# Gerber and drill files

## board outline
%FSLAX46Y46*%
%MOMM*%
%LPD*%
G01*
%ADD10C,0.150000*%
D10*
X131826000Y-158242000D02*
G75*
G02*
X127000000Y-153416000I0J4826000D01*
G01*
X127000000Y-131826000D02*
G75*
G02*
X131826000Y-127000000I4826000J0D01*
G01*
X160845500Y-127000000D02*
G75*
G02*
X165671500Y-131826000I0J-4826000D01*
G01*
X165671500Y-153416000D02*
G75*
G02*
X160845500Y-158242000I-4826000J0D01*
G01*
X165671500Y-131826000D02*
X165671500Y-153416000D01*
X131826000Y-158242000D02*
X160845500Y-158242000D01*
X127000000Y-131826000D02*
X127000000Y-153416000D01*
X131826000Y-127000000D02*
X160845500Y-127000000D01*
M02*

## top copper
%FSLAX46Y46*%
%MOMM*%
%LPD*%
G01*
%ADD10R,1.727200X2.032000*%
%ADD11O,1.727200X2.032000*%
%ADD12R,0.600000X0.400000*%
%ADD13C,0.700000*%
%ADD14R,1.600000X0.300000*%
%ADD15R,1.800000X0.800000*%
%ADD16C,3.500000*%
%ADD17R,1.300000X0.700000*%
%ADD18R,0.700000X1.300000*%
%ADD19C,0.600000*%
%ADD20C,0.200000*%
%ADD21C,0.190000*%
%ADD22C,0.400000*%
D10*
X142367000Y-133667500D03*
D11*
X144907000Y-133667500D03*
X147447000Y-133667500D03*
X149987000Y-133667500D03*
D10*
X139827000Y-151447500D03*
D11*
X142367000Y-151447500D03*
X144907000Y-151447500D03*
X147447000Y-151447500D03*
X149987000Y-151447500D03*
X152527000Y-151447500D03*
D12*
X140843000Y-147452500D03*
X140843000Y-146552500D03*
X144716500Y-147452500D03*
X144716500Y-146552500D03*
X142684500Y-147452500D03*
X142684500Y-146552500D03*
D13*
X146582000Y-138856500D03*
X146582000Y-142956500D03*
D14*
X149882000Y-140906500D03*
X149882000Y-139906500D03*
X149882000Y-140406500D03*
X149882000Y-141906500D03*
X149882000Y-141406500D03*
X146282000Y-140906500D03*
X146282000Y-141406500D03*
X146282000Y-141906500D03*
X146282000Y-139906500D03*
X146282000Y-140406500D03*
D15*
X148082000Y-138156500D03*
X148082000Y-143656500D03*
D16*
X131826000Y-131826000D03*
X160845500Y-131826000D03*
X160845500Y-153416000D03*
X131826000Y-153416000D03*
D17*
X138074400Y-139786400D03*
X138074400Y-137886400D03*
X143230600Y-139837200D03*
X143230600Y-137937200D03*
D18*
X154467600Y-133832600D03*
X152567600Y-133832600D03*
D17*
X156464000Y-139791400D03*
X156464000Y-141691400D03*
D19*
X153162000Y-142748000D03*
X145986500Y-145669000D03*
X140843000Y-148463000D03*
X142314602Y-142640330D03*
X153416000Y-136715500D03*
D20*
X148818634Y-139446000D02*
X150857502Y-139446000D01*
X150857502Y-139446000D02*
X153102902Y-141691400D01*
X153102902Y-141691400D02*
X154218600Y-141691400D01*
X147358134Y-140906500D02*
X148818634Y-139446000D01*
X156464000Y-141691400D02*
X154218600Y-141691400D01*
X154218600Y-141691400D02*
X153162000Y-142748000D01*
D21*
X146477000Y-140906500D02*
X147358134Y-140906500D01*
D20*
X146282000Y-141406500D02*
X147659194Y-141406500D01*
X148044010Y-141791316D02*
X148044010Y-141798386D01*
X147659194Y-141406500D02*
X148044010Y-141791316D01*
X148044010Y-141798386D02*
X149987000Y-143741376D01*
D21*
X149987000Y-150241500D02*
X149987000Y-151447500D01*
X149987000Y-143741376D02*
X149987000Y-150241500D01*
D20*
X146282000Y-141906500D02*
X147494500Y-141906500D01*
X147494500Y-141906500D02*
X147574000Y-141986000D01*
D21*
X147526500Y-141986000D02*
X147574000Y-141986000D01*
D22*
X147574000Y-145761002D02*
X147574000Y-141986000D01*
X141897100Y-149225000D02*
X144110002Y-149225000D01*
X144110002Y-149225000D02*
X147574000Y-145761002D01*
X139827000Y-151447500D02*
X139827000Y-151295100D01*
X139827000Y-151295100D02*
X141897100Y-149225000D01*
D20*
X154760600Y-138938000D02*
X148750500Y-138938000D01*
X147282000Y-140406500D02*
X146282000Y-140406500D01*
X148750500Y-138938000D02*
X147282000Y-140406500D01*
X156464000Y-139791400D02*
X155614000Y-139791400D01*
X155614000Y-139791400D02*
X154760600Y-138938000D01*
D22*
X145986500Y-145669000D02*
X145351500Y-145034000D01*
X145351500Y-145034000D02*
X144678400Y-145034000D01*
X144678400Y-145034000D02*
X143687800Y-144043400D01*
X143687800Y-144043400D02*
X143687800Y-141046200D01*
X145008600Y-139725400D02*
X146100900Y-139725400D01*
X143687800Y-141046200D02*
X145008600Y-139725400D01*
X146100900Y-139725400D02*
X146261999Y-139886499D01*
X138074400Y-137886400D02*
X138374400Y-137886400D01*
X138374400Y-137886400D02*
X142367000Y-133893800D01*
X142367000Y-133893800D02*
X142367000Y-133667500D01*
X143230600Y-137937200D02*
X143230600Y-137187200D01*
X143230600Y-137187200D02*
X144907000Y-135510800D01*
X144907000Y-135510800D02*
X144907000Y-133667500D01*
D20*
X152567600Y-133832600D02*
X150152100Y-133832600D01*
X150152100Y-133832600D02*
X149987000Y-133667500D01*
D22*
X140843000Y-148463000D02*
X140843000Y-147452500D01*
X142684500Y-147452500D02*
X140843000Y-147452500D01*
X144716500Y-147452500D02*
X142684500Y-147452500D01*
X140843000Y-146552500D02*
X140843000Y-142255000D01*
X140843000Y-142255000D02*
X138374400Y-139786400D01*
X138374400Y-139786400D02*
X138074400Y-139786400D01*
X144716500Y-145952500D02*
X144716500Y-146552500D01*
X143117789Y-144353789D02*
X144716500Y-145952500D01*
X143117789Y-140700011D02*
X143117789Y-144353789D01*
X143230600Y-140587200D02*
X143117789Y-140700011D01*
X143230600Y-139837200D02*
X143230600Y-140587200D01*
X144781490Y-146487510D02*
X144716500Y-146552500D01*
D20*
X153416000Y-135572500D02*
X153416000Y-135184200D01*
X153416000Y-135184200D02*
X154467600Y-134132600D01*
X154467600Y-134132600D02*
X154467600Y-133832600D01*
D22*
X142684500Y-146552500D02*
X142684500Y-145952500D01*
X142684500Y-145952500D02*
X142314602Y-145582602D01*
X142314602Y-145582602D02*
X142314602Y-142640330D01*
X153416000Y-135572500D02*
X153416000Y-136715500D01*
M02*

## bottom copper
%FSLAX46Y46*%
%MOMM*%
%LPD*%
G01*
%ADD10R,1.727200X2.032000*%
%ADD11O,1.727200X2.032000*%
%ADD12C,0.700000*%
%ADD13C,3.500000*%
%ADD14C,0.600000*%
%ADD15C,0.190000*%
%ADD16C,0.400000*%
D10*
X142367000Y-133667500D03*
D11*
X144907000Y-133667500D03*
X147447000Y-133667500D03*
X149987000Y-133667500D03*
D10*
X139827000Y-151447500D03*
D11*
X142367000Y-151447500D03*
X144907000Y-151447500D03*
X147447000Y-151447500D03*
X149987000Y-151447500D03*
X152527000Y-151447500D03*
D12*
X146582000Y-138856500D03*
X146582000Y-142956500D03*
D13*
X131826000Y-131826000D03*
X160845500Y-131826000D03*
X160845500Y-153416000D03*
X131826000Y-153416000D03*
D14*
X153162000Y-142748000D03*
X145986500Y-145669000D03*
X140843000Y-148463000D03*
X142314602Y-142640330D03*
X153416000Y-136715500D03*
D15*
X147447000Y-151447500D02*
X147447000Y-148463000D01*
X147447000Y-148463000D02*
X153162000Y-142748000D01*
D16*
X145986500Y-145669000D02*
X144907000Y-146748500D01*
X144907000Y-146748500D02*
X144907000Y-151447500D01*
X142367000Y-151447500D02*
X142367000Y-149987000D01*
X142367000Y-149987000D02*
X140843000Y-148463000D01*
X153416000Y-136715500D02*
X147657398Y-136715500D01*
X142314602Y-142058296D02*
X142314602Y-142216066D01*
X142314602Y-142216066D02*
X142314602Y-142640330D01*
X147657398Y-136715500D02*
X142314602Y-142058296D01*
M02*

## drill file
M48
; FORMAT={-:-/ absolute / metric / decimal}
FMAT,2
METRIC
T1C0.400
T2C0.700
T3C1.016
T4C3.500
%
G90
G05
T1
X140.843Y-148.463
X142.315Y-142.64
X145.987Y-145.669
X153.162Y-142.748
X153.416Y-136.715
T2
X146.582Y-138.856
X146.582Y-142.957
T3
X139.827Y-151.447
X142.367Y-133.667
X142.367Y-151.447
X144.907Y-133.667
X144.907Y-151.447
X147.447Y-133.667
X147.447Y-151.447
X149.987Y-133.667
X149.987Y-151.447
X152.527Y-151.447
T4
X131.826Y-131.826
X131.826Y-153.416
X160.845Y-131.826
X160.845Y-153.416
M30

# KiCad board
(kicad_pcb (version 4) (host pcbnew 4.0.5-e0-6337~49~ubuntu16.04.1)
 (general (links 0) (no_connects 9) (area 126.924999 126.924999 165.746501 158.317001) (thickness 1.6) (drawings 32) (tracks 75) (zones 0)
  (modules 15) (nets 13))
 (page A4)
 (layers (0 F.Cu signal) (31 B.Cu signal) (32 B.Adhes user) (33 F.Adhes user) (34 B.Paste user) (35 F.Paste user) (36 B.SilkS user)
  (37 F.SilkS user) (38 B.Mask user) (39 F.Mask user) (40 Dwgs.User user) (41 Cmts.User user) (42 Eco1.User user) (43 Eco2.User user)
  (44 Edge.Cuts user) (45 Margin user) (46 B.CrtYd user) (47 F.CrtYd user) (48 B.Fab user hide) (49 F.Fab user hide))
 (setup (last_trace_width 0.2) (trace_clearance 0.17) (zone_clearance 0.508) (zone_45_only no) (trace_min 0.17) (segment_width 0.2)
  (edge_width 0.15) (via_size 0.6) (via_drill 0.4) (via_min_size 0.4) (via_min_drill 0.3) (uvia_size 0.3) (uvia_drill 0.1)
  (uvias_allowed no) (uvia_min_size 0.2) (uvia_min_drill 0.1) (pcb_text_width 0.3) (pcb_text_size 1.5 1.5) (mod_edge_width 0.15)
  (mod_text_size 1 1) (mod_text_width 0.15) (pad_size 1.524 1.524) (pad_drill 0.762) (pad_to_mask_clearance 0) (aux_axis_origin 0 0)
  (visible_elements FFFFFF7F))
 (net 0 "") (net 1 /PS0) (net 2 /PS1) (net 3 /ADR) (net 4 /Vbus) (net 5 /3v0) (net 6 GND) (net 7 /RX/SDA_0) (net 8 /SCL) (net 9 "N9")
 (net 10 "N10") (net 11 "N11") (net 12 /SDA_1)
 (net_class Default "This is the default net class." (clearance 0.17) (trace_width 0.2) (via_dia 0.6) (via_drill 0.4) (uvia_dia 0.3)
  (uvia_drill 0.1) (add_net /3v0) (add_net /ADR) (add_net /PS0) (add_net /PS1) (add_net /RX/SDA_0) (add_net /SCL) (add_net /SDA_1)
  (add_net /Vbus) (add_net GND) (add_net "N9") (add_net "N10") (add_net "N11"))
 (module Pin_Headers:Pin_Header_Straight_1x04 (layer F.Cu) (at 142.367 133.6675 90)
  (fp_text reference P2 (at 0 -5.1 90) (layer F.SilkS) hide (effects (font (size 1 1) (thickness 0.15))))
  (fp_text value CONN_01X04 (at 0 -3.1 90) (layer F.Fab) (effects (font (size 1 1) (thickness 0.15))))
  (pad 1 thru_hole rect (at 0 0 90) (size 2.032 1.7272) (drill 1.016) (layers *.Cu *.Mask) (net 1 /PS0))
  (pad 2 thru_hole oval (at 0 2.54 90) (size 2.032 1.7272) (drill 1.016) (layers *.Cu *.Mask) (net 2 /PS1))
  (pad 3 thru_hole oval (at 0 5.08 90) (size 2.032 1.7272) (drill 1.016) (layers *.Cu *.Mask))
  (pad 4 thru_hole oval (at 0 7.62 90) (size 2.032 1.7272) (drill 1.016) (layers *.Cu *.Mask) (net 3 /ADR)))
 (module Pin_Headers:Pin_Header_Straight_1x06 (layer F.Cu) (at 139.827 151.4475 90)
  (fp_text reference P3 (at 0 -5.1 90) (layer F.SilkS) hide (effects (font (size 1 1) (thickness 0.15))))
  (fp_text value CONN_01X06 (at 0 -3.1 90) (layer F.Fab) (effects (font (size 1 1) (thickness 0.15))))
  (pad 1 thru_hole rect (at 0 0 90) (size 2.032 1.7272) (drill 1.016) (layers *.Cu *.Mask) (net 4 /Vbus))
  (pad 2 thru_hole oval (at 0 2.54 90) (size 2.032 1.7272) (drill 1.016) (layers *.Cu *.Mask) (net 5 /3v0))
  (pad 3 thru_hole oval (at 0 5.08 90) (size 2.032 1.7272) (drill 1.016) (layers *.Cu *.Mask) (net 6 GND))
  (pad 4 thru_hole oval (at 0 7.62 90) (size 2.032 1.7272) (drill 1.016) (layers *.Cu *.Mask) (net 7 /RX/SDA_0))
  (pad 5 thru_hole oval (at 0 10.16 90) (size 2.032 1.7272) (drill 1.016) (layers *.Cu *.Mask) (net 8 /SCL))
  (pad 6 thru_hole oval (at 0 12.7 90) (size 2.032 1.7272) (drill 1.016) (layers *.Cu *.Mask)))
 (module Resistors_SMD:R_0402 (layer F.Cu) (at 140.843 147.0025 90)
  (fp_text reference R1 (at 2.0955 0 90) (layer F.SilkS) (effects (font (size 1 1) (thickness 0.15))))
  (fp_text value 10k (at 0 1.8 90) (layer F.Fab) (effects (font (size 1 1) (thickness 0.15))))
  (pad 1 smd rect (at -0.45 0 90) (size 0.4 0.6) (layers F.Cu F.Paste F.Mask) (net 5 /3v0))
  (pad 2 smd rect (at 0.45 0 90) (size 0.4 0.6) (layers F.Cu F.Paste F.Mask) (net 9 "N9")))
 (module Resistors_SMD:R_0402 (layer F.Cu) (at 144.7165 147.0025 90)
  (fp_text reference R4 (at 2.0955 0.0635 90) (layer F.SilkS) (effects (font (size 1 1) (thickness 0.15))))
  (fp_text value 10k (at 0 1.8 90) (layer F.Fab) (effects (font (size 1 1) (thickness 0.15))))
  (pad 1 smd rect (at -0.45 0 90) (size 0.4 0.6) (layers F.Cu F.Paste F.Mask) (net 5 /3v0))
  (pad 2 smd rect (at 0.45 0 90) (size 0.4 0.6) (layers F.Cu F.Paste F.Mask) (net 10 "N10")))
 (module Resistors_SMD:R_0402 (layer F.Cu) (at 142.6845 147.0025 90)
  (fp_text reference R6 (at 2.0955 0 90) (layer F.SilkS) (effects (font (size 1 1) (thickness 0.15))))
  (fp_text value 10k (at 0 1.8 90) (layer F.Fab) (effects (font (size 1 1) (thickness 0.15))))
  (pad 1 smd rect (at -0.45 0 90) (size 0.4 0.6) (layers F.Cu F.Paste F.Mask) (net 5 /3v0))
  (pad 2 smd rect (at 0.45 0 90) (size 0.4 0.6) (layers F.Cu F.Paste F.Mask) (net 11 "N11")))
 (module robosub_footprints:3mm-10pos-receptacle (layer F.Cu) (at 148.082 140.9065 90)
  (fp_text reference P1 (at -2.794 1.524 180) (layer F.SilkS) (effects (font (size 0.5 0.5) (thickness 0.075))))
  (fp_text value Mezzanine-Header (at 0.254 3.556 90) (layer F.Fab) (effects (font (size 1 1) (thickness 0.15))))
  (pad "" thru_hole circle (at 2.05 -1.5 90) (size 0.7 0.7) (drill 0.7) (layers *.Cu *.Mask))
  (pad "" thru_hole circle (at -2.05 -1.5 90) (size 0.7 0.7) (drill 0.7) (layers *.Cu *.Mask))
  (pad 6 smd rect (at 0 1.8 90) (size 0.3 1.6) (layers F.Cu F.Paste F.Mask))
  (pad 10 smd rect (at 1 1.8 90) (size 0.3 1.6) (layers F.Cu F.Paste F.Mask))
  (pad 8 smd rect (at 0.5 1.8 90) (size 0.3 1.6) (layers F.Cu F.Paste F.Mask))
  (pad 2 smd rect (at -1 1.8 90) (size 0.3 1.6) (layers F.Cu F.Paste F.Mask))
  (pad 4 smd rect (at -0.5 1.8 90) (size 0.3 1.6) (layers F.Cu F.Paste F.Mask))
  (pad 5 smd rect (at 0 -1.8 90) (size 0.3 1.6) (layers F.Cu F.Paste F.Mask) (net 7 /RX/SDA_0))
  (pad 3 smd rect (at -0.5 -1.8 90) (size 0.3 1.6) (layers F.Cu F.Paste F.Mask) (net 8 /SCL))
  (pad 1 smd rect (at -1 -1.8 90) (size 0.3 1.6) (layers F.Cu F.Paste F.Mask) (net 4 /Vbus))
  (pad 9 smd rect (at 1 -1.8 90) (size 0.3 1.6) (layers F.Cu F.Paste F.Mask) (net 6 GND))
  (pad 7 smd rect (at 0.5 -1.8 90) (size 0.3 1.6) (layers F.Cu F.Paste F.Mask) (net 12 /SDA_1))
  (pad "" smd rect (at 2.75 0 90) (size 0.8 1.8) (layers F.Cu F.Paste F.Mask))
  (pad "" smd rect (at -2.75 0 90) (size 0.8 1.8) (layers F.Cu F.Paste F.Mask)))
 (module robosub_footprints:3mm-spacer (layer F.Cu) (at 131.826 131.826)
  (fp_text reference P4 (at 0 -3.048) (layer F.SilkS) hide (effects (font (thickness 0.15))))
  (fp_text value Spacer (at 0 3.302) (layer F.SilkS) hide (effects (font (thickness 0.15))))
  (pad "" thru_hole circle (at 0 0) (size 3.5 3.5) (drill 3.5) (layers *.Cu *.Mask F.SilkS)))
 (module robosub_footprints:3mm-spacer (layer F.Cu) (at 160.8455 131.826)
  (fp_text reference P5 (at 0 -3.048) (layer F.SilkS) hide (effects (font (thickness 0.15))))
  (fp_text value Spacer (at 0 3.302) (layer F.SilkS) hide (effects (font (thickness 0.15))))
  (pad "" thru_hole circle (at 0 0) (size 3.5 3.5) (drill 3.5) (layers *.Cu *.Mask F.SilkS)))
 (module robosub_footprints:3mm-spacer (layer F.Cu) (at 160.8455 153.416)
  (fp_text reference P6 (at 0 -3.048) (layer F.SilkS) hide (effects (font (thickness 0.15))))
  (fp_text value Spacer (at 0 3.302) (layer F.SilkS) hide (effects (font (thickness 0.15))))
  (pad "" thru_hole circle (at 0 0) (size 3.5 3.5) (drill 3.5) (layers *.Cu *.Mask F.SilkS)))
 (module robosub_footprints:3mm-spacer (layer F.Cu) (at 131.826 153.416)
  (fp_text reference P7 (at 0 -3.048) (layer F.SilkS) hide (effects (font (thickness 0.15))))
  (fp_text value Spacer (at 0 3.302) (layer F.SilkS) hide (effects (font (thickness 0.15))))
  (pad "" thru_hole circle (at 0 0) (size 3.5 3.5) (drill 3.5) (layers *.Cu *.Mask F.SilkS)))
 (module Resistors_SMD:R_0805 (layer F.Cu) (at 138.0744 138.8364 90)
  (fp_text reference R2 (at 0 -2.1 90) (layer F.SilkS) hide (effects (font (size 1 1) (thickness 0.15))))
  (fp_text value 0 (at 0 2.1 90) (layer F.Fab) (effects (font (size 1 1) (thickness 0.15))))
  (pad 1 smd rect (at -0.95 0 90) (size 0.7 1.3) (layers F.Cu F.Paste F.Mask) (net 9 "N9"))
  (pad 2 smd rect (at 0.95 0 90) (size 0.7 1.3) (layers F.Cu F.Paste F.Mask) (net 1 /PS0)))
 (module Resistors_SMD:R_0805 (layer F.Cu) (at 143.2306 138.8872 90)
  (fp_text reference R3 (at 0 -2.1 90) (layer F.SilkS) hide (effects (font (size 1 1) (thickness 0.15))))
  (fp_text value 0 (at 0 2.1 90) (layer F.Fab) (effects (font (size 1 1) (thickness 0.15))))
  (pad 1 smd rect (at -0.95 0 90) (size 0.7 1.3) (layers F.Cu F.Paste F.Mask) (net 10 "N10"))
  (pad 2 smd rect (at 0.95 0 90) (size 0.7 1.3) (layers F.Cu F.Paste F.Mask) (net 2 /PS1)))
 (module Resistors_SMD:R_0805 (layer F.Cu) (at 153.5176 133.8326 180)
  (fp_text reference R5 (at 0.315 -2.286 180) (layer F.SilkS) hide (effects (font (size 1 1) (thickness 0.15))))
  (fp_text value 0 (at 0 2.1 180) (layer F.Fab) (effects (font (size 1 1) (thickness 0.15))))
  (pad 1 smd rect (at -0.95 0 180) (size 0.7 1.3) (layers F.Cu F.Paste F.Mask) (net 11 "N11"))
  (pad 2 smd rect (at 0.95 0 180) (size 0.7 1.3) (layers F.Cu F.Paste F.Mask) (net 3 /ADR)))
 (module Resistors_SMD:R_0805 (layer F.Cu) (at 156.464 140.7414 270)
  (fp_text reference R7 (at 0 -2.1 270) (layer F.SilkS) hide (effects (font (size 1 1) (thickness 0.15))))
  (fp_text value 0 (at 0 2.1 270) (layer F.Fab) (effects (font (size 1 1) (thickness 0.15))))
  (pad 1 smd rect (at -0.95 0 270) (size 0.7 1.3) (layers F.Cu F.Paste F.Mask) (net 12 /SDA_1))
  (pad 2 smd rect (at 0.95 0 270) (size 0.7 1.3) (layers F.Cu F.Paste F.Mask) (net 7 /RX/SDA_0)))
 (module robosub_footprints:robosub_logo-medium (layer F.Cu) (at 162.3314 142.5702 90)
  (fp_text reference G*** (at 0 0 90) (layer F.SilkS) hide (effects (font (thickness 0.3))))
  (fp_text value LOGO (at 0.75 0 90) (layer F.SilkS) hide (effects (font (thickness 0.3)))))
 (gr_arc (start 131.826 153.416) (end 131.826 158.242) (angle 90) (layer Edge.Cuts) (width 0.15))
 (gr_arc (start 131.826 131.826) (end 127 131.826) (angle 90) (layer Edge.Cuts) (width 0.15))
 (gr_arc (start 160.8455 131.826) (end 160.8455 127) (angle 90) (layer Edge.Cuts) (width 0.15))
 (gr_arc (start 160.8455 153.416) (end 165.6715 153.416) (angle 90) (layer Edge.Cuts) (width 0.15))
 (gr_line (start 165.6715 131.826) (end 165.6715 153.416) (layer Edge.Cuts) (width 0.15))
 (gr_line (start 131.826 158.242) (end 160.8455 158.242) (layer Edge.Cuts) (width 0.15))
 (gr_line (start 127 131.826) (end 127 153.416) (layer Edge.Cuts) (width 0.15))
 (gr_line (start 131.826 127) (end 160.8455 127) (layer Edge.Cuts) (width 0.15))
 (segment (start 148.818634 139.446) (end 150.857502 139.446) (width 0.2) (layer F.Cu) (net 7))
 (segment (start 150.857502 139.446) (end 153.102902 141.6914) (width 0.2) (layer F.Cu) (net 7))
 (segment (start 153.102902 141.6914) (end 154.2186 141.6914) (width 0.2) (layer F.Cu) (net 7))
 (segment (start 147.358134 140.9065) (end 148.818634 139.446) (width 0.2) (layer F.Cu) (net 7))
 (segment (start 156.464 141.6914) (end 154.2186 141.6914) (width 0.2) (layer F.Cu) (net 7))
 (segment (start 154.2186 141.6914) (end 153.162 142.748) (width 0.2) (layer F.Cu) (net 7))
 (segment (start 147.447 151.4475) (end 147.447 148.463) (width 0.19) (layer B.Cu) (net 7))
 (segment (start 147.447 148.463) (end 153.162 142.748) (width 0.19) (layer B.Cu) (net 7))
 (via (at 153.162 142.748) (size 0.6) (drill 0.4) (layers F.Cu B.Cu) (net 7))
 (segment (start 146.477 140.9065) (end 147.358134 140.9065) (width 0.19) (layer F.Cu) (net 7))
 (segment (start 146.282 141.4065) (end 147.659194 141.4065) (width 0.2) (layer F.Cu) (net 8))
 (segment (start 148.04401 141.791316) (end 148.04401 141.798386) (width 0.2) (layer F.Cu) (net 8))
 (segment (start 147.659194 141.4065) (end 148.04401 141.791316) (width 0.2) (layer F.Cu) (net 8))
 (segment (start 148.04401 141.798386) (end 149.987 143.741376) (width 0.2) (layer F.Cu) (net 8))
 (segment (start 149.987 150.2415) (end 149.987 151.4475) (width 0.19) (layer F.Cu) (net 8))
 (segment (start 149.987 143.741376) (end 149.987 150.2415) (width 0.19) (layer F.Cu) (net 8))
 (segment (start 146.282 141.9065) (end 147.4945 141.9065) (width 0.2) (layer F.Cu) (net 4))
 (segment (start 147.4945 141.9065) (end 147.574 141.986) (width 0.2) (layer F.Cu) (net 4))
 (segment (start 147.5265 141.986) (end 147.574 141.986) (width 0.19) (layer F.Cu) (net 4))
 (segment (start 147.574 145.761002) (end 147.574 141.986) (width 0.4) (layer F.Cu) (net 4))
 (segment (start 141.8971 149.225) (end 144.110002 149.225) (width 0.4) (layer F.Cu) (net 4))
 (segment (start 144.110002 149.225) (end 147.574 145.761002) (width 0.4) (layer F.Cu) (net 4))
 (segment (start 139.827 151.4475) (end 139.827 151.2951) (width 0.4) (layer F.Cu) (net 4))
 (segment (start 139.827 151.2951) (end 141.8971 149.225) (width 0.4) (layer F.Cu) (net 4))
 (segment (start 154.7606 138.938) (end 148.7505 138.938) (width 0.2) (layer F.Cu) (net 12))
 (segment (start 147.282 140.4065) (end 146.282 140.4065) (width 0.2) (layer F.Cu) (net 12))
 (segment (start 148.7505 138.938) (end 147.282 140.4065) (width 0.2) (layer F.Cu) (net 12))
 (segment (start 156.464 139.7914) (end 155.614 139.7914) (width 0.2) (layer F.Cu) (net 12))
 (segment (start 155.614 139.7914) (end 154.7606 138.938) (width 0.2) (layer F.Cu) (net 12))
 (segment (start 145.9865 145.669) (end 145.3515 145.034) (width 0.4) (layer F.Cu) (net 6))
 (segment (start 145.3515 145.034) (end 144.6784 145.034) (width 0.4) (layer F.Cu) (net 6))
 (segment (start 144.6784 145.034) (end 143.6878 144.0434) (width 0.4) (layer F.Cu) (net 6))
 (segment (start 143.6878 144.0434) (end 143.6878 141.0462) (width 0.4) (layer F.Cu) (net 6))
 (segment (start 145.0086 139.7254) (end 146.1009 139.7254) (width 0.4) (layer F.Cu) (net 6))
 (segment (start 143.6878 141.0462) (end 145.0086 139.7254) (width 0.4) (layer F.Cu) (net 6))
 (segment (start 146.1009 139.7254) (end 146.261999 139.886499) (width 0.4) (layer F.Cu) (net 6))
 (segment (start 145.9865 145.669) (end 144.907 146.7485) (width 0.4) (layer B.Cu) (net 6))
 (segment (start 144.907 146.7485) (end 144.907 151.4475) (width 0.4) (layer B.Cu) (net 6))
 (via (at 145.9865 145.669) (size 0.6) (drill 0.4) (layers F.Cu B.Cu) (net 6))
 (segment (start 138.0744 137.8864) (end 138.3744 137.8864) (width 0.4) (layer F.Cu) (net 1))
 (segment (start 138.3744 137.8864) (end 142.367 133.8938) (width 0.4) (layer F.Cu) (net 1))
 (segment (start 142.367 133.8938) (end 142.367 133.6675) (width 0.4) (layer F.Cu) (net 1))
 (segment (start 143.2306 137.9372) (end 143.2306 137.1872) (width 0.4) (layer F.Cu) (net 2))
 (segment (start 143.2306 137.1872) (end 144.907 135.5108) (width 0.4) (layer F.Cu) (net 2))
 (segment (start 144.907 135.5108) (end 144.907 133.6675) (width 0.4) (layer F.Cu) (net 2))
 (segment (start 152.5676 133.8326) (end 150.1521 133.8326) (width 0.2) (layer F.Cu) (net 3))
 (segment (start 150.1521 133.8326) (end 149.987 133.6675) (width 0.2) (layer F.Cu) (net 3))
 (segment (start 140.843 148.463) (end 140.843 147.4525) (width 0.4) (layer F.Cu) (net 5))
 (segment (start 142.367 151.4475) (end 142.367 149.987) (width 0.4) (layer B.Cu) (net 5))
 (segment (start 142.367 149.987) (end 140.843 148.463) (width 0.4) (layer B.Cu) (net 5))
 (via (at 140.843 148.463) (size 0.6) (drill 0.4) (layers F.Cu B.Cu) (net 5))
 (segment (start 142.6845 147.4525) (end 140.843 147.4525) (width 0.4) (layer F.Cu) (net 5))
 (segment (start 144.7165 147.4525) (end 142.6845 147.4525) (width 0.4) (layer F.Cu) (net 5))
 (segment (start 140.843 146.5525) (end 140.843 142.255) (width 0.4) (layer F.Cu) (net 9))
 (segment (start 140.843 142.255) (end 138.3744 139.7864) (width 0.4) (layer F.Cu) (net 9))
 (segment (start 138.3744 139.7864) (end 138.0744 139.7864) (width 0.4) (layer F.Cu) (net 9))
 (segment (start 144.7165 145.9525) (end 144.7165 146.5525) (width 0.4) (layer F.Cu) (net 10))
 (segment (start 143.117789 144.353789) (end 144.7165 145.9525) (width 0.4) (layer F.Cu) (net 10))
 (segment (start 143.117789 140.700011) (end 143.117789 144.353789) (width 0.4) (layer F.Cu) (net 10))
 (segment (start 143.2306 140.5872) (end 143.117789 140.700011) (width 0.4) (layer F.Cu) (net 10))
 (segment (start 143.2306 139.8372) (end 143.2306 140.5872) (width 0.4) (layer F.Cu) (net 10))
 (segment (start 144.78149 146.48751) (end 144.7165 146.5525) (width 0.4) (layer F.Cu) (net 10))
 (segment (start 153.416 135.5725) (end 153.416 135.1842) (width 0.2) (layer F.Cu) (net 11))
 (segment (start 153.416 135.1842) (end 154.4676 134.1326) (width 0.2) (layer F.Cu) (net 11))
 (segment (start 154.4676 134.1326) (end 154.4676 133.8326) (width 0.2) (layer F.Cu) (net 11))
 (segment (start 153.416 136.7155) (end 147.657398 136.7155) (width 0.4) (layer B.Cu) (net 11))
 (segment (start 142.314602 142.058296) (end 142.314602 142.216066) (width 0.4) (layer B.Cu) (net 11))
 (via (at 142.314602 142.64033) (size 0.6) (drill 0.4) (layers F.Cu B.Cu) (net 11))
 (segment (start 142.314602 142.216066) (end 142.314602 142.64033) (width 0.4) (layer B.Cu) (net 11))
 (segment (start 147.657398 136.7155) (end 142.314602 142.058296) (width 0.4) (layer B.Cu) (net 11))
 (segment (start 142.6845 146.5525) (end 142.6845 145.9525) (width 0.4) (layer F.Cu) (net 11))
 (segment (start 142.6845 145.9525) (end 142.314602 145.582602) (width 0.4) (layer F.Cu) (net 11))
 (segment (start 142.314602 145.582602) (end 142.314602 142.64033) (width 0.4) (layer F.Cu) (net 11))
 (segment (start 153.416 135.5725) (end 153.416 136.7155) (width 0.4) (layer F.Cu) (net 11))
 (via (at 153.416 136.7155) (size 0.6) (drill 0.4) (layers F.Cu B.Cu) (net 11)))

